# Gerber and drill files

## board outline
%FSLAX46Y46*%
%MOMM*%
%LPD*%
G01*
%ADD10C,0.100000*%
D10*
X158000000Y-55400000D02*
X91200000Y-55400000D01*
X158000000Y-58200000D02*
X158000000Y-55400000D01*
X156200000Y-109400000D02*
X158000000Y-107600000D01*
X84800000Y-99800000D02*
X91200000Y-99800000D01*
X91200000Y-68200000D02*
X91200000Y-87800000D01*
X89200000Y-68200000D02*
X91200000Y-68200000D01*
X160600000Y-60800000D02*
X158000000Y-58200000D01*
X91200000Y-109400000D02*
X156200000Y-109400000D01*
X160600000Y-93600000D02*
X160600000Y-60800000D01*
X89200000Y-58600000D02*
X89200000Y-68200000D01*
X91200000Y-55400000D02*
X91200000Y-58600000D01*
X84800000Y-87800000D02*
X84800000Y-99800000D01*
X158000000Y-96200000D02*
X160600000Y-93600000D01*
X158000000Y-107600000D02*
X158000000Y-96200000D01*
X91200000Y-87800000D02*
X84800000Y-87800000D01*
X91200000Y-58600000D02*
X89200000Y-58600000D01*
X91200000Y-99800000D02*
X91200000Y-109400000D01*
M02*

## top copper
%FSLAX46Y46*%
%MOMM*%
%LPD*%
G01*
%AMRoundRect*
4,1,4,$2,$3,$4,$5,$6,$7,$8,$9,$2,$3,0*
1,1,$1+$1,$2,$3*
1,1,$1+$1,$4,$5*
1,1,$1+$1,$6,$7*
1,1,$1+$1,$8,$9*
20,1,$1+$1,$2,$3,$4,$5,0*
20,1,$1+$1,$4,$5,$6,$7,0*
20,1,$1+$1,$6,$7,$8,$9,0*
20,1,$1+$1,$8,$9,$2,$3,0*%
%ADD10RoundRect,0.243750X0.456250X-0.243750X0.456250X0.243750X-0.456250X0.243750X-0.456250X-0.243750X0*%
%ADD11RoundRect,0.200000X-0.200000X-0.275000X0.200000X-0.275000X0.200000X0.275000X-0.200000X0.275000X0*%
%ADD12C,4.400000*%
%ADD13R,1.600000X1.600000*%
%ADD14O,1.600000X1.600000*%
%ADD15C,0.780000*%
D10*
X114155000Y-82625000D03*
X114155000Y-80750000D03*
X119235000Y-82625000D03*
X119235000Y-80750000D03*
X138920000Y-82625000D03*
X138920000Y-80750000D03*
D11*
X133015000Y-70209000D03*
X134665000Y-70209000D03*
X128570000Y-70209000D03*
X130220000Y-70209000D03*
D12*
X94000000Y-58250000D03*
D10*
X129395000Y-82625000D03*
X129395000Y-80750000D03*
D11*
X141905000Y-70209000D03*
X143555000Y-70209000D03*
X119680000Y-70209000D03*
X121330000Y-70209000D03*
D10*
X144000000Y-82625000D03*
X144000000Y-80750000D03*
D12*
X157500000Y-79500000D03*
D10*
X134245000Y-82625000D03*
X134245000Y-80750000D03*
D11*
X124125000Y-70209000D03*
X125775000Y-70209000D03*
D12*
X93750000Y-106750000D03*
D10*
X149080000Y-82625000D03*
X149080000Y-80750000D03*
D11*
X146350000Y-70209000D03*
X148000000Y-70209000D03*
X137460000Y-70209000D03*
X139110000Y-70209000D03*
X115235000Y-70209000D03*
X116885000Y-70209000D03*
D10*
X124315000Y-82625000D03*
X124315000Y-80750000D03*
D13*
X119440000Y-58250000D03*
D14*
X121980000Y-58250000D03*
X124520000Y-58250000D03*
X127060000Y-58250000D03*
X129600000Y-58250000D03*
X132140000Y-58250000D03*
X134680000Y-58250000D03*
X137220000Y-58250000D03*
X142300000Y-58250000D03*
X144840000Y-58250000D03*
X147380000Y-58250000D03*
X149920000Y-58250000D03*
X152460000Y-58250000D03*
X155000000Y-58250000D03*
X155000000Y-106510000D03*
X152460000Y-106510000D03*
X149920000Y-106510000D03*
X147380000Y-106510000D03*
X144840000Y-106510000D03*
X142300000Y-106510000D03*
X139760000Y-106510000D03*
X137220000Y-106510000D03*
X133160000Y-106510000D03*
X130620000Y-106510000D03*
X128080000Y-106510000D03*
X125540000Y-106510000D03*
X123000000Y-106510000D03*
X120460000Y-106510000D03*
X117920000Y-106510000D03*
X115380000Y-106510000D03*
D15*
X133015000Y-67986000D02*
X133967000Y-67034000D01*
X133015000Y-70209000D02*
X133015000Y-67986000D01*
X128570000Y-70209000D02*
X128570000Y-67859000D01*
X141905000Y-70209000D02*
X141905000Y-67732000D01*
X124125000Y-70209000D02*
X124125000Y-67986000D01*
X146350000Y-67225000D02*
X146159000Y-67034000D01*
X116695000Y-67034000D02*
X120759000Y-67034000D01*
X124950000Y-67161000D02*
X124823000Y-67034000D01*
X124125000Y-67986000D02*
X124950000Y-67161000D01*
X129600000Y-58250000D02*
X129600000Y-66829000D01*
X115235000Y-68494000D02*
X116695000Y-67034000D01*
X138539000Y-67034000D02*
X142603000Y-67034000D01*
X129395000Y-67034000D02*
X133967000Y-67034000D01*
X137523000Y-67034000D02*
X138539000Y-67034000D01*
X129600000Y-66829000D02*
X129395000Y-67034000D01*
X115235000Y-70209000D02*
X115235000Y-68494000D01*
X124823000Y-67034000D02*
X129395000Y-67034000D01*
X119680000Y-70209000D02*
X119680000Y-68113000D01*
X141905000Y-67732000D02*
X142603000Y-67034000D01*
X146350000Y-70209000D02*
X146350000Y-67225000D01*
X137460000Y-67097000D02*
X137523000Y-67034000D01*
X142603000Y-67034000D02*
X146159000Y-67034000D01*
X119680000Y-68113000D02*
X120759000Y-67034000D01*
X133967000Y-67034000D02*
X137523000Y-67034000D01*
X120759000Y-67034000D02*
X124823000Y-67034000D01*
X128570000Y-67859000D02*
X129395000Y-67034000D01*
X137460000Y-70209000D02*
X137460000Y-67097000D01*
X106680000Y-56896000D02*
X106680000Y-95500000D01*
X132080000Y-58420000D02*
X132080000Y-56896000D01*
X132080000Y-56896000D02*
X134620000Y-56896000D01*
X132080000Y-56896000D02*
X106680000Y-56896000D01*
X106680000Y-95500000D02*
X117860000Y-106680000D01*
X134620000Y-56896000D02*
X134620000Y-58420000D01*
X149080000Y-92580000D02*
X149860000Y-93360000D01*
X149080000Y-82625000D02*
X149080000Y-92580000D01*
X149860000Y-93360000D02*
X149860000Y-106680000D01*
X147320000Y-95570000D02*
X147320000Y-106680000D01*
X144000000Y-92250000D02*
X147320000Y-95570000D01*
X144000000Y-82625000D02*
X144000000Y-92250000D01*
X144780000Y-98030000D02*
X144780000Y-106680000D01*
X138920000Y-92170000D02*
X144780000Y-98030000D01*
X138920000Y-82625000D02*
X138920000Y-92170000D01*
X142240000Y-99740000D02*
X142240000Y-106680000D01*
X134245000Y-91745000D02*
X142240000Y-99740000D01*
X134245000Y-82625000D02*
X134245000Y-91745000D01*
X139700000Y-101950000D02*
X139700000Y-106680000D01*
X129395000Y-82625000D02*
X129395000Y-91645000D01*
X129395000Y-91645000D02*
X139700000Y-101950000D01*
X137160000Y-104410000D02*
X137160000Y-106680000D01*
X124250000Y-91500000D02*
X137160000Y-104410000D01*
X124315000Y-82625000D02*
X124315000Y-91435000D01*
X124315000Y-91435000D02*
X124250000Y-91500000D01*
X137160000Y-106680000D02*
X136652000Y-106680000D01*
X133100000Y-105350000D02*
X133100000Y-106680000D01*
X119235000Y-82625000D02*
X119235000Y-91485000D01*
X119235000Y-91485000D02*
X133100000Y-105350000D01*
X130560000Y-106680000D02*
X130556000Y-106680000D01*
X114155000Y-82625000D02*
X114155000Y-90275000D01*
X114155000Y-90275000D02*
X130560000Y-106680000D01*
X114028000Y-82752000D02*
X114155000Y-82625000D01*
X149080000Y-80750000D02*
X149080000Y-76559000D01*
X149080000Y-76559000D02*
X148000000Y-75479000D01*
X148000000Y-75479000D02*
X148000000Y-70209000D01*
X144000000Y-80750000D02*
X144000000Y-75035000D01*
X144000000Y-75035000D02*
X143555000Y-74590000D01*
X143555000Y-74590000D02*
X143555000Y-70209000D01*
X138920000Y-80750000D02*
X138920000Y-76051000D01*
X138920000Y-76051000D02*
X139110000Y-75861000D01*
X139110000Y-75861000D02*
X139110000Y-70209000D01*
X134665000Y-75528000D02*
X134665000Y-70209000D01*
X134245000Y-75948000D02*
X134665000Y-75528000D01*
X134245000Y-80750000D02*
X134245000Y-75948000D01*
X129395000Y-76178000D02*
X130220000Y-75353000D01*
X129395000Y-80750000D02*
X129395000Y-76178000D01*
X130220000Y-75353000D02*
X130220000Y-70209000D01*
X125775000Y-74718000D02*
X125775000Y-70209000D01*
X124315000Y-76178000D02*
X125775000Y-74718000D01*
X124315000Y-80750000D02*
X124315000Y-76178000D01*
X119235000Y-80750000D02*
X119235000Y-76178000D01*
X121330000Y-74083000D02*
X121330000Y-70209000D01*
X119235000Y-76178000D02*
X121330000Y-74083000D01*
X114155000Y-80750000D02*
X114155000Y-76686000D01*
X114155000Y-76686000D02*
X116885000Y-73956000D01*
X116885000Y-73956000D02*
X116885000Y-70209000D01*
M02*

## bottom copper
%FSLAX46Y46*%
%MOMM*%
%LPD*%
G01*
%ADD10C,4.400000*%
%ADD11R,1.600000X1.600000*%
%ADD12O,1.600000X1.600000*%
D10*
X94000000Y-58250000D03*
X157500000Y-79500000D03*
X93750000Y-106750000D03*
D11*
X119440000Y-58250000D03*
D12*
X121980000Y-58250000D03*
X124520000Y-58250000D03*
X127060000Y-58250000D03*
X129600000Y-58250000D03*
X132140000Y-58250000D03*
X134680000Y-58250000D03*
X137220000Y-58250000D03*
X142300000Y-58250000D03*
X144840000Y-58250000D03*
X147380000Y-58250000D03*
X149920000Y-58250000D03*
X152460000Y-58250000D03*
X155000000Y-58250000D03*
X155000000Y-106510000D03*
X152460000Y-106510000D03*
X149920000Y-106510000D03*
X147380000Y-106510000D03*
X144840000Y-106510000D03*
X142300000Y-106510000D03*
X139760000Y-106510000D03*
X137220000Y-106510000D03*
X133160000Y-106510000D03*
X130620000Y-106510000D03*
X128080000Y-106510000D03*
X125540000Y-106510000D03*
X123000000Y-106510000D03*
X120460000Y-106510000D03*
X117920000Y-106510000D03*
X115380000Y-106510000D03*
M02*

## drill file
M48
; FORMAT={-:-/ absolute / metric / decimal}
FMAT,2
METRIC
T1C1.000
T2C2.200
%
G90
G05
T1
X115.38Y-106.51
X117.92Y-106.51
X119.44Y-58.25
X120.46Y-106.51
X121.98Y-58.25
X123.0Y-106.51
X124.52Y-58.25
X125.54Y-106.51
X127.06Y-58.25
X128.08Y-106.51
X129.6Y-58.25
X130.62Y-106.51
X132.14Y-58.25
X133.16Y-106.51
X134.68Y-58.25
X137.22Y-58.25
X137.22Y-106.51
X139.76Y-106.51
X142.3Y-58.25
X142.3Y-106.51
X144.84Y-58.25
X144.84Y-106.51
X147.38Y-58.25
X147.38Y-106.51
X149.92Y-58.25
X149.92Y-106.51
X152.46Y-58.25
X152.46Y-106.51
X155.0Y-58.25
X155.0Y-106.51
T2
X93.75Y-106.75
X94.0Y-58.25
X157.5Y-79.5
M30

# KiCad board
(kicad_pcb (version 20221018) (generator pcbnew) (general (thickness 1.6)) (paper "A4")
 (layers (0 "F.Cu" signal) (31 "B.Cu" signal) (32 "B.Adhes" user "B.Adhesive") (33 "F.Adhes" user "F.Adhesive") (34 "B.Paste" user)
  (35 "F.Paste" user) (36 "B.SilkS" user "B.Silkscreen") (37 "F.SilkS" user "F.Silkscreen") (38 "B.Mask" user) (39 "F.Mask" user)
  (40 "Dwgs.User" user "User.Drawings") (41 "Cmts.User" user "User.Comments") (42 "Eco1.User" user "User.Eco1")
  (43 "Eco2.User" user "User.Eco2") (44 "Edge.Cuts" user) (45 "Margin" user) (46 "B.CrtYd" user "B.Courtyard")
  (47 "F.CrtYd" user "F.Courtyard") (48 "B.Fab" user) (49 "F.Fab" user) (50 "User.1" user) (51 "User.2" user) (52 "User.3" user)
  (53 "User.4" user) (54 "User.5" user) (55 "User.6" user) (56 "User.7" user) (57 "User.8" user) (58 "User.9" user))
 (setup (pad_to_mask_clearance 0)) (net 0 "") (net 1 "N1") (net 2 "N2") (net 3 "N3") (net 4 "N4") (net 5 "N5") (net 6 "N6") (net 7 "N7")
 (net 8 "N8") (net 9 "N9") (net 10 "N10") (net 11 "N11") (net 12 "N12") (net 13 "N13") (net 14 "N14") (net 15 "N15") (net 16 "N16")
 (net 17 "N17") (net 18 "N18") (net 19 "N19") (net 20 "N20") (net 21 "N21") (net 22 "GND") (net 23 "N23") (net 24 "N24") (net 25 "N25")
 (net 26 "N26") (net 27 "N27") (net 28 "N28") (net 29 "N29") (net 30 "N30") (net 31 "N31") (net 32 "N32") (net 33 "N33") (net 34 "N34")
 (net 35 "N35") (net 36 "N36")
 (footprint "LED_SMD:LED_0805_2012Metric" (layer "F.Cu") (at 114.155 81.6875 90)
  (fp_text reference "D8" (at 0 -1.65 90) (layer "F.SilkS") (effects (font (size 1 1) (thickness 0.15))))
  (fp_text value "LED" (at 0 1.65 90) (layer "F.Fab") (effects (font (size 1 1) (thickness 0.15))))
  (pad "1" smd roundrect (at -0.9375 0 90) (size 0.975 1.4) (layers "F.Cu" "F.Paste" "F.Mask") (roundrect_rratio 0.25) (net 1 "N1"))
  (pad "2" smd roundrect (at 0.9375 0 90) (size 0.975 1.4) (layers "F.Cu" "F.Paste" "F.Mask") (roundrect_rratio 0.25) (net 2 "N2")))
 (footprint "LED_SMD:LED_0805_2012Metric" (layer "F.Cu") (at 119.235 81.6875 90)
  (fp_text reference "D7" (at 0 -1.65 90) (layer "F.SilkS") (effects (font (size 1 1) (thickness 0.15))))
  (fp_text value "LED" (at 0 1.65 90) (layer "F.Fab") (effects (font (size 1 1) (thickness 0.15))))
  (pad "1" smd roundrect (at -0.9375 0 90) (size 0.975 1.4) (layers "F.Cu" "F.Paste" "F.Mask") (roundrect_rratio 0.25) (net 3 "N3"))
  (pad "2" smd roundrect (at 0.9375 0 90) (size 0.975 1.4) (layers "F.Cu" "F.Paste" "F.Mask") (roundrect_rratio 0.25) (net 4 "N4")))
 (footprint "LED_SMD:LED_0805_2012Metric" (layer "F.Cu") (at 138.92 81.6875 90)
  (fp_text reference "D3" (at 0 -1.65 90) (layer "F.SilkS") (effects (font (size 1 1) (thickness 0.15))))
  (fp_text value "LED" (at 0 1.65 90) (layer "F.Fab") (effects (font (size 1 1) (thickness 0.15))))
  (pad "1" smd roundrect (at -0.9375 0 90) (size 0.975 1.4) (layers "F.Cu" "F.Paste" "F.Mask") (roundrect_rratio 0.25) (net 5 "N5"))
  (pad "2" smd roundrect (at 0.9375 0 90) (size 0.975 1.4) (layers "F.Cu" "F.Paste" "F.Mask") (roundrect_rratio 0.25) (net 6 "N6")))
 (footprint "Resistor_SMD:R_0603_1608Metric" (layer "F.Cu") (at 133.84 70.209)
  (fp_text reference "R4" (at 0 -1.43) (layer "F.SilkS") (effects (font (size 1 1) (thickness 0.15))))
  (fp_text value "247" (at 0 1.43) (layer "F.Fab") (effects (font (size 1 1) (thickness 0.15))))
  (pad "1" smd roundrect (at -0.825 0) (size 0.8 0.95) (layers "F.Cu" "F.Paste" "F.Mask") (roundrect_rratio 0.25) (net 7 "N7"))
  (pad "2" smd roundrect (at 0.825 0) (size 0.8 0.95) (layers "F.Cu" "F.Paste" "F.Mask") (roundrect_rratio 0.25) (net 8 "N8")))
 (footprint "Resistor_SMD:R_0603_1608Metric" (layer "F.Cu") (at 129.395 70.209)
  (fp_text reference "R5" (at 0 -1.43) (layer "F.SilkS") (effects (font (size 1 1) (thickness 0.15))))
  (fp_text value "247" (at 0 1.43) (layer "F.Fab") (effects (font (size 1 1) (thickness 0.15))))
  (pad "1" smd roundrect (at -0.825 0) (size 0.8 0.95) (layers "F.Cu" "F.Paste" "F.Mask") (roundrect_rratio 0.25) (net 7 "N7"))
  (pad "2" smd roundrect (at 0.825 0) (size 0.8 0.95) (layers "F.Cu" "F.Paste" "F.Mask") (roundrect_rratio 0.25) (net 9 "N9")))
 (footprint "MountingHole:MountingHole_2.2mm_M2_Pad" (layer "F.Cu") (at 94 58.25)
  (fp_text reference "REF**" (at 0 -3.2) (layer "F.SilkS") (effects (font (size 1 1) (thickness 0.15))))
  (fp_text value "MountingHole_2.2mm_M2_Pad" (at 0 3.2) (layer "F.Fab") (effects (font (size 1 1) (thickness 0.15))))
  (pad "1" thru_hole circle (at 0 0) (size 4.4 4.4) (drill 2.2) (layers "*.Cu" "*.Mask")))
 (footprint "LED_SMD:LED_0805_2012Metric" (layer "F.Cu") (at 129.395 81.6875 90)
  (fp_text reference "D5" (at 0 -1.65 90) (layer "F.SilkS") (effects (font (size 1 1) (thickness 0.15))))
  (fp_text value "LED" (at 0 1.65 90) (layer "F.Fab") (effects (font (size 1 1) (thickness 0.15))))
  (pad "1" smd roundrect (at -0.9375 0 90) (size 0.975 1.4) (layers "F.Cu" "F.Paste" "F.Mask") (roundrect_rratio 0.25) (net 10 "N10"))
  (pad "2" smd roundrect (at 0.9375 0 90) (size 0.975 1.4) (layers "F.Cu" "F.Paste" "F.Mask") (roundrect_rratio 0.25) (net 9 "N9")))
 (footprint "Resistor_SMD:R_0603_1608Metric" (layer "F.Cu") (at 142.73 70.209)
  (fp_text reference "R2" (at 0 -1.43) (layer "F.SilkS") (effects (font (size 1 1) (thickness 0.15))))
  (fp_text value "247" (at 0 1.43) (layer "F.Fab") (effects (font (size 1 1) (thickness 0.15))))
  (pad "1" smd roundrect (at -0.825 0) (size 0.8 0.95) (layers "F.Cu" "F.Paste" "F.Mask") (roundrect_rratio 0.25) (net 7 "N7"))
  (pad "2" smd roundrect (at 0.825 0) (size 0.8 0.95) (layers "F.Cu" "F.Paste" "F.Mask") (roundrect_rratio 0.25) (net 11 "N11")))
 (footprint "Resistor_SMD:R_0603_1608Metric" (layer "F.Cu") (at 120.505 70.209)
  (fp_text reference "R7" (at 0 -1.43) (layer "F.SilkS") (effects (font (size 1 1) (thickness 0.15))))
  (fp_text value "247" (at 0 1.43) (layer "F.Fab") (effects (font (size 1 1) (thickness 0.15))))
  (pad "1" smd roundrect (at -0.825 0) (size 0.8 0.95) (layers "F.Cu" "F.Paste" "F.Mask") (roundrect_rratio 0.25) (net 7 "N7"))
  (pad "2" smd roundrect (at 0.825 0) (size 0.8 0.95) (layers "F.Cu" "F.Paste" "F.Mask") (roundrect_rratio 0.25) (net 4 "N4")))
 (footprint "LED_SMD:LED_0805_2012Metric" (layer "F.Cu") (at 144 81.6875 90)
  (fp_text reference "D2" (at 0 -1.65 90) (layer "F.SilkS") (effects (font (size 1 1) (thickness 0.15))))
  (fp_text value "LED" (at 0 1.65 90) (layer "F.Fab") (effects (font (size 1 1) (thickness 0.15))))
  (pad "1" smd roundrect (at -0.9375 0 90) (size 0.975 1.4) (layers "F.Cu" "F.Paste" "F.Mask") (roundrect_rratio 0.25) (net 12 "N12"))
  (pad "2" smd roundrect (at 0.9375 0 90) (size 0.975 1.4) (layers "F.Cu" "F.Paste" "F.Mask") (roundrect_rratio 0.25) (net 11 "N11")))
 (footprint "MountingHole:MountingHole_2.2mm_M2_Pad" (layer "F.Cu") (at 157.5 79.5)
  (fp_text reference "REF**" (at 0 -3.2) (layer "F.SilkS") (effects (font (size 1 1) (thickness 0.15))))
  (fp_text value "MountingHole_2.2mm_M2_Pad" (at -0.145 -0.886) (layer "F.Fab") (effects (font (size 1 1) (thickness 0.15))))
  (pad "1" thru_hole circle (at 0 0) (size 4.4 4.4) (drill 2.2) (layers "*.Cu" "*.Mask")))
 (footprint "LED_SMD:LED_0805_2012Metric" (layer "F.Cu") (at 134.245 81.6875 90)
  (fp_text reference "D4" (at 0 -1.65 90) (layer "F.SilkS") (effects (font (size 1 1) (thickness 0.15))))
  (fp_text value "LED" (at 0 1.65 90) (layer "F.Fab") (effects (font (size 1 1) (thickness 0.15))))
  (pad "1" smd roundrect (at -0.9375 0 90) (size 0.975 1.4) (layers "F.Cu" "F.Paste" "F.Mask") (roundrect_rratio 0.25) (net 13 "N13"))
  (pad "2" smd roundrect (at 0.9375 0 90) (size 0.975 1.4) (layers "F.Cu" "F.Paste" "F.Mask") (roundrect_rratio 0.25) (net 8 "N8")))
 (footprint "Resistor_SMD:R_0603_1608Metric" (layer "F.Cu") (at 124.95 70.209)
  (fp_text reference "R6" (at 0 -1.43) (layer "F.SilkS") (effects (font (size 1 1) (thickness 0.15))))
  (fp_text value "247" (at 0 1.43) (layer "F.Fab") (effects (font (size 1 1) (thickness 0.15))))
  (pad "1" smd roundrect (at -0.825 0) (size 0.8 0.95) (layers "F.Cu" "F.Paste" "F.Mask") (roundrect_rratio 0.25) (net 7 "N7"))
  (pad "2" smd roundrect (at 0.825 0) (size 0.8 0.95) (layers "F.Cu" "F.Paste" "F.Mask") (roundrect_rratio 0.25) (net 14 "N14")))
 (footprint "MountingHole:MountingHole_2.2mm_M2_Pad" (layer "F.Cu") (at 93.75 106.75)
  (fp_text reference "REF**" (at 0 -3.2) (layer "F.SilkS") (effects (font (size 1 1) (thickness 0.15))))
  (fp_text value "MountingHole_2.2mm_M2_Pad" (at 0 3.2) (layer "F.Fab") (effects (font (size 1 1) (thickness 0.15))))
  (pad "1" thru_hole circle (at 0 0) (size 4.4 4.4) (drill 2.2) (layers "*.Cu" "*.Mask")))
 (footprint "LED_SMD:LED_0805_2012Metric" (layer "F.Cu") (at 149.08 81.6875 90)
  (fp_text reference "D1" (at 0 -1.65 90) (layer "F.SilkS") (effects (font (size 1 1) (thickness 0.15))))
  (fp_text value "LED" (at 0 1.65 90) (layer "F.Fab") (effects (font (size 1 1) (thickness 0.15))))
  (pad "1" smd roundrect (at -0.9375 0 90) (size 0.975 1.4) (layers "F.Cu" "F.Paste" "F.Mask") (roundrect_rratio 0.25) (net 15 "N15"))
  (pad "2" smd roundrect (at 0.9375 0 90) (size 0.975 1.4) (layers "F.Cu" "F.Paste" "F.Mask") (roundrect_rratio 0.25) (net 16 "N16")))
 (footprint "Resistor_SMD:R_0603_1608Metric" (layer "F.Cu") (at 147.175 70.209)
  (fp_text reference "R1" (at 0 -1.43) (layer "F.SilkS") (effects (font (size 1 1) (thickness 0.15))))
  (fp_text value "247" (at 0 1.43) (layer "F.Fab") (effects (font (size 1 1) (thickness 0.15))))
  (pad "1" smd roundrect (at -0.825 0) (size 0.8 0.95) (layers "F.Cu" "F.Paste" "F.Mask") (roundrect_rratio 0.25) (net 7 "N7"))
  (pad "2" smd roundrect (at 0.825 0) (size 0.8 0.95) (layers "F.Cu" "F.Paste" "F.Mask") (roundrect_rratio 0.25) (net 16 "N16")))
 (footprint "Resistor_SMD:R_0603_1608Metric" (layer "F.Cu") (at 138.285 70.209)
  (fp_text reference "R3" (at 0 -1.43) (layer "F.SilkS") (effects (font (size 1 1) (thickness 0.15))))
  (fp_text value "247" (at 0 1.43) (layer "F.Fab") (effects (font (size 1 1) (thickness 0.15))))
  (pad "1" smd roundrect (at -0.825 0) (size 0.8 0.95) (layers "F.Cu" "F.Paste" "F.Mask") (roundrect_rratio 0.25) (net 7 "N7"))
  (pad "2" smd roundrect (at 0.825 0) (size 0.8 0.95) (layers "F.Cu" "F.Paste" "F.Mask") (roundrect_rratio 0.25) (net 6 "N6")))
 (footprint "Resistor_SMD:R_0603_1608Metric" (layer "F.Cu") (at 116.06 70.209)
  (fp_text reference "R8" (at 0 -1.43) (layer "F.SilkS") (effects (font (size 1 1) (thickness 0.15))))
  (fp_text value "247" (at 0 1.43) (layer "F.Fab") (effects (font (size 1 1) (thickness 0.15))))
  (pad "1" smd roundrect (at -0.825 0) (size 0.8 0.95) (layers "F.Cu" "F.Paste" "F.Mask") (roundrect_rratio 0.25) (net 7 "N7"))
  (pad "2" smd roundrect (at 0.825 0) (size 0.8 0.95) (layers "F.Cu" "F.Paste" "F.Mask") (roundrect_rratio 0.25) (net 2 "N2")))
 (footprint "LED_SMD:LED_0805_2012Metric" (layer "F.Cu") (at 124.315 81.6875 90)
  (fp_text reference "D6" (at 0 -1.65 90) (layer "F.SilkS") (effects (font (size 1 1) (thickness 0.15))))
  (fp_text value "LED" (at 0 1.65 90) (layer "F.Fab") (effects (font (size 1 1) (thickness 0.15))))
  (pad "1" smd roundrect (at -0.9375 0 90) (size 0.975 1.4) (layers "F.Cu" "F.Paste" "F.Mask") (roundrect_rratio 0.25) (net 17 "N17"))
  (pad "2" smd roundrect (at 0.9375 0 90) (size 0.975 1.4) (layers "F.Cu" "F.Paste" "F.Mask") (roundrect_rratio 0.25) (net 14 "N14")))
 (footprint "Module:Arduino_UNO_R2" (layer "F.Cu") (at 119.44 58.25)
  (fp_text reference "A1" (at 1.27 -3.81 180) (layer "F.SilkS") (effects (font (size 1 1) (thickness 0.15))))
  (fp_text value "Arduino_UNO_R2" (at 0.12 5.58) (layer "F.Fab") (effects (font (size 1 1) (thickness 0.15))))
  (pad "1" thru_hole rect (at 0 0 90) (size 1.6 1.6) (drill 1) (layers "*.Cu" "*.Mask") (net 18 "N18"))
  (pad "2" thru_hole oval (at 2.54 0 90) (size 1.6 1.6) (drill 1) (layers "*.Cu" "*.Mask") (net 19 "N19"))
  (pad "3" thru_hole oval (at 5.08 0 90) (size 1.6 1.6) (drill 1) (layers "*.Cu" "*.Mask") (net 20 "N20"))
  (pad "4" thru_hole oval (at 7.62 0 90) (size 1.6 1.6) (drill 1) (layers "*.Cu" "*.Mask") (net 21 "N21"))
  (pad "5" thru_hole oval (at 10.16 0 90) (size 1.6 1.6) (drill 1) (layers "*.Cu" "*.Mask") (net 7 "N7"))
  (pad "6" thru_hole oval (at 12.7 0 90) (size 1.6 1.6) (drill 1) (layers "*.Cu" "*.Mask") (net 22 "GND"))
  (pad "7" thru_hole oval (at 15.24 0 90) (size 1.6 1.6) (drill 1) (layers "*.Cu" "*.Mask") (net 22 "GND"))
  (pad "8" thru_hole oval (at 17.78 0 90) (size 1.6 1.6) (drill 1) (layers "*.Cu" "*.Mask") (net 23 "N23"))
  (pad "9" thru_hole oval (at 22.86 0 90) (size 1.6 1.6) (drill 1) (layers "*.Cu" "*.Mask") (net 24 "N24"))
  (pad "10" thru_hole oval (at 25.4 0 90) (size 1.6 1.6) (drill 1) (layers "*.Cu" "*.Mask") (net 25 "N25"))
  (pad "11" thru_hole oval (at 27.94 0 90) (size 1.6 1.6) (drill 1) (layers "*.Cu" "*.Mask") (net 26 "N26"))
  (pad "12" thru_hole oval (at 30.48 0 90) (size 1.6 1.6) (drill 1) (layers "*.Cu" "*.Mask") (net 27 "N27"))
  (pad "13" thru_hole oval (at 33.02 0 90) (size 1.6 1.6) (drill 1) (layers "*.Cu" "*.Mask") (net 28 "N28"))
  (pad "14" thru_hole oval (at 35.56 0 90) (size 1.6 1.6) (drill 1) (layers "*.Cu" "*.Mask") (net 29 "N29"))
  (pad "15" thru_hole oval (at 35.56 48.26 90) (size 1.6 1.6) (drill 1) (layers "*.Cu" "*.Mask") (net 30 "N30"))
  (pad "16" thru_hole oval (at 33.02 48.26 90) (size 1.6 1.6) (drill 1) (layers "*.Cu" "*.Mask") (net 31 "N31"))
  (pad "17" thru_hole oval (at 30.48 48.26 90) (size 1.6 1.6) (drill 1) (layers "*.Cu" "*.Mask") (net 15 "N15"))
  (pad "18" thru_hole oval (at 27.94 48.26 90) (size 1.6 1.6) (drill 1) (layers "*.Cu" "*.Mask") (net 12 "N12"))
  (pad "19" thru_hole oval (at 25.4 48.26 90) (size 1.6 1.6) (drill 1) (layers "*.Cu" "*.Mask") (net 5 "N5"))
  (pad "20" thru_hole oval (at 22.86 48.26 90) (size 1.6 1.6) (drill 1) (layers "*.Cu" "*.Mask") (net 13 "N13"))
  (pad "21" thru_hole oval (at 20.32 48.26 90) (size 1.6 1.6) (drill 1) (layers "*.Cu" "*.Mask") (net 10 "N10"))
  (pad "22" thru_hole oval (at 17.78 48.26 90) (size 1.6 1.6) (drill 1) (layers "*.Cu" "*.Mask") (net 17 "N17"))
  (pad "23" thru_hole oval (at 13.72 48.26 90) (size 1.6 1.6) (drill 1) (layers "*.Cu" "*.Mask") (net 3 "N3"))
  (pad "24" thru_hole oval (at 11.18 48.26 90) (size 1.6 1.6) (drill 1) (layers "*.Cu" "*.Mask") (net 1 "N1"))
  (pad "25" thru_hole oval (at 8.64 48.26 90) (size 1.6 1.6) (drill 1) (layers "*.Cu" "*.Mask") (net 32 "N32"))
  (pad "26" thru_hole oval (at 6.1 48.26 90) (size 1.6 1.6) (drill 1) (layers "*.Cu" "*.Mask") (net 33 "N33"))
  (pad "27" thru_hole oval (at 3.56 48.26 90) (size 1.6 1.6) (drill 1) (layers "*.Cu" "*.Mask") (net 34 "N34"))
  (pad "28" thru_hole oval (at 1.02 48.26 90) (size 1.6 1.6) (drill 1) (layers "*.Cu" "*.Mask") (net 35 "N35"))
  (pad "29" thru_hole oval (at -1.52 48.26 90) (size 1.6 1.6) (drill 1) (layers "*.Cu" "*.Mask") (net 22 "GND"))
  (pad "30" thru_hole oval (at -4.06 48.26 90) (size 1.6 1.6) (drill 1) (layers "*.Cu" "*.Mask") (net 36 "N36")))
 (gr_line (start 158 55.4) (end 91.2 55.4) (stroke (width 0.1) (type default)) (layer "Edge.Cuts"))
 (gr_line (start 158 58.2) (end 158 55.4) (stroke (width 0.1) (type default)) (layer "Edge.Cuts"))
 (gr_line (start 156.2 109.4) (end 158 107.6) (stroke (width 0.1) (type default)) (layer "Edge.Cuts"))
 (gr_line (start 84.8 99.8) (end 91.2 99.8) (stroke (width 0.1) (type default)) (layer "Edge.Cuts"))
 (gr_line (start 91.2 68.2) (end 91.2 87.8) (stroke (width 0.1) (type default)) (layer "Edge.Cuts"))
 (gr_line (start 89.2 68.2) (end 91.2 68.2) (stroke (width 0.1) (type default)) (layer "Edge.Cuts"))
 (gr_line (start 160.6 60.8) (end 158 58.2) (stroke (width 0.1) (type default)) (layer "Edge.Cuts"))
 (gr_line (start 91.2 109.4) (end 156.2 109.4) (stroke (width 0.1) (type default)) (layer "Edge.Cuts"))
 (gr_line (start 160.6 93.6) (end 160.6 60.8) (stroke (width 0.1) (type default)) (layer "Edge.Cuts"))
 (gr_line (start 89.2 58.6) (end 89.2 68.2) (stroke (width 0.1) (type default)) (layer "Edge.Cuts"))
 (gr_line (start 91.2 55.4) (end 91.2 58.6) (stroke (width 0.1) (type default)) (layer "Edge.Cuts"))
 (gr_line (start 84.8 87.8) (end 84.8 99.8) (stroke (width 0.1) (type default)) (layer "Edge.Cuts"))
 (gr_line (start 158 96.2) (end 160.6 93.6) (stroke (width 0.1) (type default)) (layer "Edge.Cuts"))
 (gr_line (start 158 107.6) (end 158 96.2) (stroke (width 0.1) (type default)) (layer "Edge.Cuts"))
 (gr_line (start 91.2 87.8) (end 84.8 87.8) (stroke (width 0.1) (type default)) (layer "Edge.Cuts"))
 (gr_line (start 91.2 58.6) (end 89.2 58.6) (stroke (width 0.1) (type default)) (layer "Edge.Cuts"))
 (gr_line (start 91.2 99.8) (end 91.2 109.4) (stroke (width 0.1) (type default)) (layer "Edge.Cuts"))
 (segment (start 133.015 67.986) (end 133.967 67.034) (width 0.78) (layer "F.Cu") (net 7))
 (segment (start 133.015 70.209) (end 133.015 67.986) (width 0.78) (layer "F.Cu") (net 7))
 (segment (start 128.57 70.209) (end 128.57 67.859) (width 0.78) (layer "F.Cu") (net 7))
 (segment (start 141.905 70.209) (end 141.905 67.732) (width 0.78) (layer "F.Cu") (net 7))
 (segment (start 124.125 70.209) (end 124.125 67.986) (width 0.78) (layer "F.Cu") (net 7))
 (segment (start 146.35 67.225) (end 146.159 67.034) (width 0.78) (layer "F.Cu") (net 7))
 (segment (start 116.695 67.034) (end 120.759 67.034) (width 0.78) (layer "F.Cu") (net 7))
 (segment (start 124.95 67.161) (end 124.823 67.034) (width 0.78) (layer "F.Cu") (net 7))
 (segment (start 124.125 67.986) (end 124.95 67.161) (width 0.78) (layer "F.Cu") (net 7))
 (segment (start 129.6 58.25) (end 129.6 66.829) (width 0.78) (layer "F.Cu") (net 7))
 (segment (start 115.235 68.494) (end 116.695 67.034) (width 0.78) (layer "F.Cu") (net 7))
 (segment (start 138.539 67.034) (end 142.603 67.034) (width 0.78) (layer "F.Cu") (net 7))
 (segment (start 129.395 67.034) (end 133.967 67.034) (width 0.78) (layer "F.Cu") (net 7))
 (segment (start 137.523 67.034) (end 138.539 67.034) (width 0.78) (layer "F.Cu") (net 7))
 (segment (start 129.6 66.829) (end 129.395 67.034) (width 0.78) (layer "F.Cu") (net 7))
 (segment (start 115.235 70.209) (end 115.235 68.494) (width 0.78) (layer "F.Cu") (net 7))
 (segment (start 124.823 67.034) (end 129.395 67.034) (width 0.78) (layer "F.Cu") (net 7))
 (segment (start 119.68 70.209) (end 119.68 68.113) (width 0.78) (layer "F.Cu") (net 7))
 (segment (start 141.905 67.732) (end 142.603 67.034) (width 0.78) (layer "F.Cu") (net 7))
 (segment (start 146.35 70.209) (end 146.35 67.225) (width 0.78) (layer "F.Cu") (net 7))
 (segment (start 137.46 67.097) (end 137.523 67.034) (width 0.78) (layer "F.Cu") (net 7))
 (segment (start 142.603 67.034) (end 146.159 67.034) (width 0.78) (layer "F.Cu") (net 7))
 (segment (start 119.68 68.113) (end 120.759 67.034) (width 0.78) (layer "F.Cu") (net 7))
 (segment (start 133.967 67.034) (end 137.523 67.034) (width 0.78) (layer "F.Cu") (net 7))
 (segment (start 120.759 67.034) (end 124.823 67.034) (width 0.78) (layer "F.Cu") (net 7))
 (segment (start 128.57 67.859) (end 129.395 67.034) (width 0.78) (layer "F.Cu") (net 7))
 (segment (start 137.46 70.209) (end 137.46 67.097) (width 0.78) (layer "F.Cu") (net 7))
 (segment (start 106.68 56.896) (end 106.68 95.5) (width 0.78) (layer "F.Cu") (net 22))
 (segment (start 132.08 58.42) (end 132.08 56.896) (width 0.78) (layer "F.Cu") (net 22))
 (segment (start 132.08 56.896) (end 134.62 56.896) (width 0.78) (layer "F.Cu") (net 22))
 (segment (start 132.08 56.896) (end 106.68 56.896) (width 0.78) (layer "F.Cu") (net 22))
 (segment (start 106.68 95.5) (end 117.86 106.68) (width 0.78) (layer "F.Cu") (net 22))
 (segment (start 134.62 56.896) (end 134.62 58.42) (width 0.78) (layer "F.Cu") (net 22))
 (segment (start 149.08 92.58) (end 149.86 93.36) (width 0.78) (layer "F.Cu") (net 15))
 (segment (start 149.08 82.625) (end 149.08 92.58) (width 0.78) (layer "F.Cu") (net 15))
 (segment (start 149.86 93.36) (end 149.86 106.68) (width 0.78) (layer "F.Cu") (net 15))
 (segment (start 147.32 95.57) (end 147.32 106.68) (width 0.78) (layer "F.Cu") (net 12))
 (segment (start 144 92.25) (end 147.32 95.57) (width 0.78) (layer "F.Cu") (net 12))
 (segment (start 144 82.625) (end 144 92.25) (width 0.78) (layer "F.Cu") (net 12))
 (segment (start 144.78 98.03) (end 144.78 106.68) (width 0.78) (layer "F.Cu") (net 5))
 (segment (start 138.92 92.17) (end 144.78 98.03) (width 0.78) (layer "F.Cu") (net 5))
 (segment (start 138.92 82.625) (end 138.92 92.17) (width 0.78) (layer "F.Cu") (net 5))
 (segment (start 142.24 99.74) (end 142.24 106.68) (width 0.78) (layer "F.Cu") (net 13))
 (segment (start 134.245 91.745) (end 142.24 99.74) (width 0.78) (layer "F.Cu") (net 13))
 (segment (start 134.245 82.625) (end 134.245 91.745) (width 0.78) (layer "F.Cu") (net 13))
 (segment (start 139.7 101.95) (end 139.7 106.68) (width 0.78) (layer "F.Cu") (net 10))
 (segment (start 129.395 82.625) (end 129.395 91.645) (width 0.78) (layer "F.Cu") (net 10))
 (segment (start 129.395 91.645) (end 139.7 101.95) (width 0.78) (layer "F.Cu") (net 10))
 (segment (start 137.16 104.41) (end 137.16 106.68) (width 0.78) (layer "F.Cu") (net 17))
 (segment (start 124.25 91.5) (end 137.16 104.41) (width 0.78) (layer "F.Cu") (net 17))
 (segment (start 124.315 82.625) (end 124.315 91.435) (width 0.78) (layer "F.Cu") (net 17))
 (segment (start 124.315 91.435) (end 124.25 91.5) (width 0.78) (layer "F.Cu") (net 17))
 (segment (start 137.16 106.68) (end 136.652 106.68) (width 0.78) (layer "F.Cu") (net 17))
 (segment (start 133.1 105.35) (end 133.1 106.68) (width 0.78) (layer "F.Cu") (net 3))
 (segment (start 119.235 82.625) (end 119.235 91.485) (width 0.78) (layer "F.Cu") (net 3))
 (segment (start 119.235 91.485) (end 133.1 105.35) (width 0.78) (layer "F.Cu") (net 3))
 (segment (start 130.56 106.68) (end 130.556 106.68) (width 0.78) (layer "F.Cu") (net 1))
 (segment (start 114.155 82.625) (end 114.155 90.275) (width 0.78) (layer "F.Cu") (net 1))
 (segment (start 114.155 90.275) (end 130.56 106.68) (width 0.78) (layer "F.Cu") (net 1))
 (segment (start 114.028 82.752) (end 114.155 82.625) (width 0.78) (layer "F.Cu") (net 1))
 (segment (start 149.08 80.75) (end 149.08 76.559) (width 0.78) (layer "F.Cu") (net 16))
 (segment (start 149.08 76.559) (end 148 75.479) (width 0.78) (layer "F.Cu") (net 16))
 (segment (start 148 75.479) (end 148 70.209) (width 0.78) (layer "F.Cu") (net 16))
 (segment (start 144 80.75) (end 144 75.035) (width 0.78) (layer "F.Cu") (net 11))
 (segment (start 144 75.035) (end 143.555 74.59) (width 0.78) (layer "F.Cu") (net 11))
 (segment (start 143.555 74.59) (end 143.555 70.209) (width 0.78) (layer "F.Cu") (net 11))
 (segment (start 138.92 80.75) (end 138.92 76.051) (width 0.78) (layer "F.Cu") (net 6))
 (segment (start 138.92 76.051) (end 139.11 75.861) (width 0.78) (layer "F.Cu") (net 6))
 (segment (start 139.11 75.861) (end 139.11 70.209) (width 0.78) (layer "F.Cu") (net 6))
 (segment (start 134.665 75.528) (end 134.665 70.209) (width 0.78) (layer "F.Cu") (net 8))
 (segment (start 134.245 75.948) (end 134.665 75.528) (width 0.78) (layer "F.Cu") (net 8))
 (segment (start 134.245 80.75) (end 134.245 75.948) (width 0.78) (layer "F.Cu") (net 8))
 (segment (start 129.395 76.178) (end 130.22 75.353) (width 0.78) (layer "F.Cu") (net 9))
 (segment (start 129.395 80.75) (end 129.395 76.178) (width 0.78) (layer "F.Cu") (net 9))
 (segment (start 130.22 75.353) (end 130.22 70.209) (width 0.78) (layer "F.Cu") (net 9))
 (segment (start 125.775 74.718) (end 125.775 70.209) (width 0.78) (layer "F.Cu") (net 14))
 (segment (start 124.315 76.178) (end 125.775 74.718) (width 0.78) (layer "F.Cu") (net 14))
 (segment (start 124.315 80.75) (end 124.315 76.178) (width 0.78) (layer "F.Cu") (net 14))
 (segment (start 119.235 80.75) (end 119.235 76.178) (width 0.78) (layer "F.Cu") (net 4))
 (segment (start 121.33 74.083) (end 121.33 70.209) (width 0.78) (layer "F.Cu") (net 4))
 (segment (start 119.235 76.178) (end 121.33 74.083) (width 0.78) (layer "F.Cu") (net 4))
 (segment (start 114.155 80.75) (end 114.155 76.686) (width 0.78) (layer "F.Cu") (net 2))
 (segment (start 114.155 76.686) (end 116.885 73.956) (width 0.78) (layer "F.Cu") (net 2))
 (segment (start 116.885 73.956) (end 116.885 70.209) (width 0.78) (layer "F.Cu") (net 2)))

